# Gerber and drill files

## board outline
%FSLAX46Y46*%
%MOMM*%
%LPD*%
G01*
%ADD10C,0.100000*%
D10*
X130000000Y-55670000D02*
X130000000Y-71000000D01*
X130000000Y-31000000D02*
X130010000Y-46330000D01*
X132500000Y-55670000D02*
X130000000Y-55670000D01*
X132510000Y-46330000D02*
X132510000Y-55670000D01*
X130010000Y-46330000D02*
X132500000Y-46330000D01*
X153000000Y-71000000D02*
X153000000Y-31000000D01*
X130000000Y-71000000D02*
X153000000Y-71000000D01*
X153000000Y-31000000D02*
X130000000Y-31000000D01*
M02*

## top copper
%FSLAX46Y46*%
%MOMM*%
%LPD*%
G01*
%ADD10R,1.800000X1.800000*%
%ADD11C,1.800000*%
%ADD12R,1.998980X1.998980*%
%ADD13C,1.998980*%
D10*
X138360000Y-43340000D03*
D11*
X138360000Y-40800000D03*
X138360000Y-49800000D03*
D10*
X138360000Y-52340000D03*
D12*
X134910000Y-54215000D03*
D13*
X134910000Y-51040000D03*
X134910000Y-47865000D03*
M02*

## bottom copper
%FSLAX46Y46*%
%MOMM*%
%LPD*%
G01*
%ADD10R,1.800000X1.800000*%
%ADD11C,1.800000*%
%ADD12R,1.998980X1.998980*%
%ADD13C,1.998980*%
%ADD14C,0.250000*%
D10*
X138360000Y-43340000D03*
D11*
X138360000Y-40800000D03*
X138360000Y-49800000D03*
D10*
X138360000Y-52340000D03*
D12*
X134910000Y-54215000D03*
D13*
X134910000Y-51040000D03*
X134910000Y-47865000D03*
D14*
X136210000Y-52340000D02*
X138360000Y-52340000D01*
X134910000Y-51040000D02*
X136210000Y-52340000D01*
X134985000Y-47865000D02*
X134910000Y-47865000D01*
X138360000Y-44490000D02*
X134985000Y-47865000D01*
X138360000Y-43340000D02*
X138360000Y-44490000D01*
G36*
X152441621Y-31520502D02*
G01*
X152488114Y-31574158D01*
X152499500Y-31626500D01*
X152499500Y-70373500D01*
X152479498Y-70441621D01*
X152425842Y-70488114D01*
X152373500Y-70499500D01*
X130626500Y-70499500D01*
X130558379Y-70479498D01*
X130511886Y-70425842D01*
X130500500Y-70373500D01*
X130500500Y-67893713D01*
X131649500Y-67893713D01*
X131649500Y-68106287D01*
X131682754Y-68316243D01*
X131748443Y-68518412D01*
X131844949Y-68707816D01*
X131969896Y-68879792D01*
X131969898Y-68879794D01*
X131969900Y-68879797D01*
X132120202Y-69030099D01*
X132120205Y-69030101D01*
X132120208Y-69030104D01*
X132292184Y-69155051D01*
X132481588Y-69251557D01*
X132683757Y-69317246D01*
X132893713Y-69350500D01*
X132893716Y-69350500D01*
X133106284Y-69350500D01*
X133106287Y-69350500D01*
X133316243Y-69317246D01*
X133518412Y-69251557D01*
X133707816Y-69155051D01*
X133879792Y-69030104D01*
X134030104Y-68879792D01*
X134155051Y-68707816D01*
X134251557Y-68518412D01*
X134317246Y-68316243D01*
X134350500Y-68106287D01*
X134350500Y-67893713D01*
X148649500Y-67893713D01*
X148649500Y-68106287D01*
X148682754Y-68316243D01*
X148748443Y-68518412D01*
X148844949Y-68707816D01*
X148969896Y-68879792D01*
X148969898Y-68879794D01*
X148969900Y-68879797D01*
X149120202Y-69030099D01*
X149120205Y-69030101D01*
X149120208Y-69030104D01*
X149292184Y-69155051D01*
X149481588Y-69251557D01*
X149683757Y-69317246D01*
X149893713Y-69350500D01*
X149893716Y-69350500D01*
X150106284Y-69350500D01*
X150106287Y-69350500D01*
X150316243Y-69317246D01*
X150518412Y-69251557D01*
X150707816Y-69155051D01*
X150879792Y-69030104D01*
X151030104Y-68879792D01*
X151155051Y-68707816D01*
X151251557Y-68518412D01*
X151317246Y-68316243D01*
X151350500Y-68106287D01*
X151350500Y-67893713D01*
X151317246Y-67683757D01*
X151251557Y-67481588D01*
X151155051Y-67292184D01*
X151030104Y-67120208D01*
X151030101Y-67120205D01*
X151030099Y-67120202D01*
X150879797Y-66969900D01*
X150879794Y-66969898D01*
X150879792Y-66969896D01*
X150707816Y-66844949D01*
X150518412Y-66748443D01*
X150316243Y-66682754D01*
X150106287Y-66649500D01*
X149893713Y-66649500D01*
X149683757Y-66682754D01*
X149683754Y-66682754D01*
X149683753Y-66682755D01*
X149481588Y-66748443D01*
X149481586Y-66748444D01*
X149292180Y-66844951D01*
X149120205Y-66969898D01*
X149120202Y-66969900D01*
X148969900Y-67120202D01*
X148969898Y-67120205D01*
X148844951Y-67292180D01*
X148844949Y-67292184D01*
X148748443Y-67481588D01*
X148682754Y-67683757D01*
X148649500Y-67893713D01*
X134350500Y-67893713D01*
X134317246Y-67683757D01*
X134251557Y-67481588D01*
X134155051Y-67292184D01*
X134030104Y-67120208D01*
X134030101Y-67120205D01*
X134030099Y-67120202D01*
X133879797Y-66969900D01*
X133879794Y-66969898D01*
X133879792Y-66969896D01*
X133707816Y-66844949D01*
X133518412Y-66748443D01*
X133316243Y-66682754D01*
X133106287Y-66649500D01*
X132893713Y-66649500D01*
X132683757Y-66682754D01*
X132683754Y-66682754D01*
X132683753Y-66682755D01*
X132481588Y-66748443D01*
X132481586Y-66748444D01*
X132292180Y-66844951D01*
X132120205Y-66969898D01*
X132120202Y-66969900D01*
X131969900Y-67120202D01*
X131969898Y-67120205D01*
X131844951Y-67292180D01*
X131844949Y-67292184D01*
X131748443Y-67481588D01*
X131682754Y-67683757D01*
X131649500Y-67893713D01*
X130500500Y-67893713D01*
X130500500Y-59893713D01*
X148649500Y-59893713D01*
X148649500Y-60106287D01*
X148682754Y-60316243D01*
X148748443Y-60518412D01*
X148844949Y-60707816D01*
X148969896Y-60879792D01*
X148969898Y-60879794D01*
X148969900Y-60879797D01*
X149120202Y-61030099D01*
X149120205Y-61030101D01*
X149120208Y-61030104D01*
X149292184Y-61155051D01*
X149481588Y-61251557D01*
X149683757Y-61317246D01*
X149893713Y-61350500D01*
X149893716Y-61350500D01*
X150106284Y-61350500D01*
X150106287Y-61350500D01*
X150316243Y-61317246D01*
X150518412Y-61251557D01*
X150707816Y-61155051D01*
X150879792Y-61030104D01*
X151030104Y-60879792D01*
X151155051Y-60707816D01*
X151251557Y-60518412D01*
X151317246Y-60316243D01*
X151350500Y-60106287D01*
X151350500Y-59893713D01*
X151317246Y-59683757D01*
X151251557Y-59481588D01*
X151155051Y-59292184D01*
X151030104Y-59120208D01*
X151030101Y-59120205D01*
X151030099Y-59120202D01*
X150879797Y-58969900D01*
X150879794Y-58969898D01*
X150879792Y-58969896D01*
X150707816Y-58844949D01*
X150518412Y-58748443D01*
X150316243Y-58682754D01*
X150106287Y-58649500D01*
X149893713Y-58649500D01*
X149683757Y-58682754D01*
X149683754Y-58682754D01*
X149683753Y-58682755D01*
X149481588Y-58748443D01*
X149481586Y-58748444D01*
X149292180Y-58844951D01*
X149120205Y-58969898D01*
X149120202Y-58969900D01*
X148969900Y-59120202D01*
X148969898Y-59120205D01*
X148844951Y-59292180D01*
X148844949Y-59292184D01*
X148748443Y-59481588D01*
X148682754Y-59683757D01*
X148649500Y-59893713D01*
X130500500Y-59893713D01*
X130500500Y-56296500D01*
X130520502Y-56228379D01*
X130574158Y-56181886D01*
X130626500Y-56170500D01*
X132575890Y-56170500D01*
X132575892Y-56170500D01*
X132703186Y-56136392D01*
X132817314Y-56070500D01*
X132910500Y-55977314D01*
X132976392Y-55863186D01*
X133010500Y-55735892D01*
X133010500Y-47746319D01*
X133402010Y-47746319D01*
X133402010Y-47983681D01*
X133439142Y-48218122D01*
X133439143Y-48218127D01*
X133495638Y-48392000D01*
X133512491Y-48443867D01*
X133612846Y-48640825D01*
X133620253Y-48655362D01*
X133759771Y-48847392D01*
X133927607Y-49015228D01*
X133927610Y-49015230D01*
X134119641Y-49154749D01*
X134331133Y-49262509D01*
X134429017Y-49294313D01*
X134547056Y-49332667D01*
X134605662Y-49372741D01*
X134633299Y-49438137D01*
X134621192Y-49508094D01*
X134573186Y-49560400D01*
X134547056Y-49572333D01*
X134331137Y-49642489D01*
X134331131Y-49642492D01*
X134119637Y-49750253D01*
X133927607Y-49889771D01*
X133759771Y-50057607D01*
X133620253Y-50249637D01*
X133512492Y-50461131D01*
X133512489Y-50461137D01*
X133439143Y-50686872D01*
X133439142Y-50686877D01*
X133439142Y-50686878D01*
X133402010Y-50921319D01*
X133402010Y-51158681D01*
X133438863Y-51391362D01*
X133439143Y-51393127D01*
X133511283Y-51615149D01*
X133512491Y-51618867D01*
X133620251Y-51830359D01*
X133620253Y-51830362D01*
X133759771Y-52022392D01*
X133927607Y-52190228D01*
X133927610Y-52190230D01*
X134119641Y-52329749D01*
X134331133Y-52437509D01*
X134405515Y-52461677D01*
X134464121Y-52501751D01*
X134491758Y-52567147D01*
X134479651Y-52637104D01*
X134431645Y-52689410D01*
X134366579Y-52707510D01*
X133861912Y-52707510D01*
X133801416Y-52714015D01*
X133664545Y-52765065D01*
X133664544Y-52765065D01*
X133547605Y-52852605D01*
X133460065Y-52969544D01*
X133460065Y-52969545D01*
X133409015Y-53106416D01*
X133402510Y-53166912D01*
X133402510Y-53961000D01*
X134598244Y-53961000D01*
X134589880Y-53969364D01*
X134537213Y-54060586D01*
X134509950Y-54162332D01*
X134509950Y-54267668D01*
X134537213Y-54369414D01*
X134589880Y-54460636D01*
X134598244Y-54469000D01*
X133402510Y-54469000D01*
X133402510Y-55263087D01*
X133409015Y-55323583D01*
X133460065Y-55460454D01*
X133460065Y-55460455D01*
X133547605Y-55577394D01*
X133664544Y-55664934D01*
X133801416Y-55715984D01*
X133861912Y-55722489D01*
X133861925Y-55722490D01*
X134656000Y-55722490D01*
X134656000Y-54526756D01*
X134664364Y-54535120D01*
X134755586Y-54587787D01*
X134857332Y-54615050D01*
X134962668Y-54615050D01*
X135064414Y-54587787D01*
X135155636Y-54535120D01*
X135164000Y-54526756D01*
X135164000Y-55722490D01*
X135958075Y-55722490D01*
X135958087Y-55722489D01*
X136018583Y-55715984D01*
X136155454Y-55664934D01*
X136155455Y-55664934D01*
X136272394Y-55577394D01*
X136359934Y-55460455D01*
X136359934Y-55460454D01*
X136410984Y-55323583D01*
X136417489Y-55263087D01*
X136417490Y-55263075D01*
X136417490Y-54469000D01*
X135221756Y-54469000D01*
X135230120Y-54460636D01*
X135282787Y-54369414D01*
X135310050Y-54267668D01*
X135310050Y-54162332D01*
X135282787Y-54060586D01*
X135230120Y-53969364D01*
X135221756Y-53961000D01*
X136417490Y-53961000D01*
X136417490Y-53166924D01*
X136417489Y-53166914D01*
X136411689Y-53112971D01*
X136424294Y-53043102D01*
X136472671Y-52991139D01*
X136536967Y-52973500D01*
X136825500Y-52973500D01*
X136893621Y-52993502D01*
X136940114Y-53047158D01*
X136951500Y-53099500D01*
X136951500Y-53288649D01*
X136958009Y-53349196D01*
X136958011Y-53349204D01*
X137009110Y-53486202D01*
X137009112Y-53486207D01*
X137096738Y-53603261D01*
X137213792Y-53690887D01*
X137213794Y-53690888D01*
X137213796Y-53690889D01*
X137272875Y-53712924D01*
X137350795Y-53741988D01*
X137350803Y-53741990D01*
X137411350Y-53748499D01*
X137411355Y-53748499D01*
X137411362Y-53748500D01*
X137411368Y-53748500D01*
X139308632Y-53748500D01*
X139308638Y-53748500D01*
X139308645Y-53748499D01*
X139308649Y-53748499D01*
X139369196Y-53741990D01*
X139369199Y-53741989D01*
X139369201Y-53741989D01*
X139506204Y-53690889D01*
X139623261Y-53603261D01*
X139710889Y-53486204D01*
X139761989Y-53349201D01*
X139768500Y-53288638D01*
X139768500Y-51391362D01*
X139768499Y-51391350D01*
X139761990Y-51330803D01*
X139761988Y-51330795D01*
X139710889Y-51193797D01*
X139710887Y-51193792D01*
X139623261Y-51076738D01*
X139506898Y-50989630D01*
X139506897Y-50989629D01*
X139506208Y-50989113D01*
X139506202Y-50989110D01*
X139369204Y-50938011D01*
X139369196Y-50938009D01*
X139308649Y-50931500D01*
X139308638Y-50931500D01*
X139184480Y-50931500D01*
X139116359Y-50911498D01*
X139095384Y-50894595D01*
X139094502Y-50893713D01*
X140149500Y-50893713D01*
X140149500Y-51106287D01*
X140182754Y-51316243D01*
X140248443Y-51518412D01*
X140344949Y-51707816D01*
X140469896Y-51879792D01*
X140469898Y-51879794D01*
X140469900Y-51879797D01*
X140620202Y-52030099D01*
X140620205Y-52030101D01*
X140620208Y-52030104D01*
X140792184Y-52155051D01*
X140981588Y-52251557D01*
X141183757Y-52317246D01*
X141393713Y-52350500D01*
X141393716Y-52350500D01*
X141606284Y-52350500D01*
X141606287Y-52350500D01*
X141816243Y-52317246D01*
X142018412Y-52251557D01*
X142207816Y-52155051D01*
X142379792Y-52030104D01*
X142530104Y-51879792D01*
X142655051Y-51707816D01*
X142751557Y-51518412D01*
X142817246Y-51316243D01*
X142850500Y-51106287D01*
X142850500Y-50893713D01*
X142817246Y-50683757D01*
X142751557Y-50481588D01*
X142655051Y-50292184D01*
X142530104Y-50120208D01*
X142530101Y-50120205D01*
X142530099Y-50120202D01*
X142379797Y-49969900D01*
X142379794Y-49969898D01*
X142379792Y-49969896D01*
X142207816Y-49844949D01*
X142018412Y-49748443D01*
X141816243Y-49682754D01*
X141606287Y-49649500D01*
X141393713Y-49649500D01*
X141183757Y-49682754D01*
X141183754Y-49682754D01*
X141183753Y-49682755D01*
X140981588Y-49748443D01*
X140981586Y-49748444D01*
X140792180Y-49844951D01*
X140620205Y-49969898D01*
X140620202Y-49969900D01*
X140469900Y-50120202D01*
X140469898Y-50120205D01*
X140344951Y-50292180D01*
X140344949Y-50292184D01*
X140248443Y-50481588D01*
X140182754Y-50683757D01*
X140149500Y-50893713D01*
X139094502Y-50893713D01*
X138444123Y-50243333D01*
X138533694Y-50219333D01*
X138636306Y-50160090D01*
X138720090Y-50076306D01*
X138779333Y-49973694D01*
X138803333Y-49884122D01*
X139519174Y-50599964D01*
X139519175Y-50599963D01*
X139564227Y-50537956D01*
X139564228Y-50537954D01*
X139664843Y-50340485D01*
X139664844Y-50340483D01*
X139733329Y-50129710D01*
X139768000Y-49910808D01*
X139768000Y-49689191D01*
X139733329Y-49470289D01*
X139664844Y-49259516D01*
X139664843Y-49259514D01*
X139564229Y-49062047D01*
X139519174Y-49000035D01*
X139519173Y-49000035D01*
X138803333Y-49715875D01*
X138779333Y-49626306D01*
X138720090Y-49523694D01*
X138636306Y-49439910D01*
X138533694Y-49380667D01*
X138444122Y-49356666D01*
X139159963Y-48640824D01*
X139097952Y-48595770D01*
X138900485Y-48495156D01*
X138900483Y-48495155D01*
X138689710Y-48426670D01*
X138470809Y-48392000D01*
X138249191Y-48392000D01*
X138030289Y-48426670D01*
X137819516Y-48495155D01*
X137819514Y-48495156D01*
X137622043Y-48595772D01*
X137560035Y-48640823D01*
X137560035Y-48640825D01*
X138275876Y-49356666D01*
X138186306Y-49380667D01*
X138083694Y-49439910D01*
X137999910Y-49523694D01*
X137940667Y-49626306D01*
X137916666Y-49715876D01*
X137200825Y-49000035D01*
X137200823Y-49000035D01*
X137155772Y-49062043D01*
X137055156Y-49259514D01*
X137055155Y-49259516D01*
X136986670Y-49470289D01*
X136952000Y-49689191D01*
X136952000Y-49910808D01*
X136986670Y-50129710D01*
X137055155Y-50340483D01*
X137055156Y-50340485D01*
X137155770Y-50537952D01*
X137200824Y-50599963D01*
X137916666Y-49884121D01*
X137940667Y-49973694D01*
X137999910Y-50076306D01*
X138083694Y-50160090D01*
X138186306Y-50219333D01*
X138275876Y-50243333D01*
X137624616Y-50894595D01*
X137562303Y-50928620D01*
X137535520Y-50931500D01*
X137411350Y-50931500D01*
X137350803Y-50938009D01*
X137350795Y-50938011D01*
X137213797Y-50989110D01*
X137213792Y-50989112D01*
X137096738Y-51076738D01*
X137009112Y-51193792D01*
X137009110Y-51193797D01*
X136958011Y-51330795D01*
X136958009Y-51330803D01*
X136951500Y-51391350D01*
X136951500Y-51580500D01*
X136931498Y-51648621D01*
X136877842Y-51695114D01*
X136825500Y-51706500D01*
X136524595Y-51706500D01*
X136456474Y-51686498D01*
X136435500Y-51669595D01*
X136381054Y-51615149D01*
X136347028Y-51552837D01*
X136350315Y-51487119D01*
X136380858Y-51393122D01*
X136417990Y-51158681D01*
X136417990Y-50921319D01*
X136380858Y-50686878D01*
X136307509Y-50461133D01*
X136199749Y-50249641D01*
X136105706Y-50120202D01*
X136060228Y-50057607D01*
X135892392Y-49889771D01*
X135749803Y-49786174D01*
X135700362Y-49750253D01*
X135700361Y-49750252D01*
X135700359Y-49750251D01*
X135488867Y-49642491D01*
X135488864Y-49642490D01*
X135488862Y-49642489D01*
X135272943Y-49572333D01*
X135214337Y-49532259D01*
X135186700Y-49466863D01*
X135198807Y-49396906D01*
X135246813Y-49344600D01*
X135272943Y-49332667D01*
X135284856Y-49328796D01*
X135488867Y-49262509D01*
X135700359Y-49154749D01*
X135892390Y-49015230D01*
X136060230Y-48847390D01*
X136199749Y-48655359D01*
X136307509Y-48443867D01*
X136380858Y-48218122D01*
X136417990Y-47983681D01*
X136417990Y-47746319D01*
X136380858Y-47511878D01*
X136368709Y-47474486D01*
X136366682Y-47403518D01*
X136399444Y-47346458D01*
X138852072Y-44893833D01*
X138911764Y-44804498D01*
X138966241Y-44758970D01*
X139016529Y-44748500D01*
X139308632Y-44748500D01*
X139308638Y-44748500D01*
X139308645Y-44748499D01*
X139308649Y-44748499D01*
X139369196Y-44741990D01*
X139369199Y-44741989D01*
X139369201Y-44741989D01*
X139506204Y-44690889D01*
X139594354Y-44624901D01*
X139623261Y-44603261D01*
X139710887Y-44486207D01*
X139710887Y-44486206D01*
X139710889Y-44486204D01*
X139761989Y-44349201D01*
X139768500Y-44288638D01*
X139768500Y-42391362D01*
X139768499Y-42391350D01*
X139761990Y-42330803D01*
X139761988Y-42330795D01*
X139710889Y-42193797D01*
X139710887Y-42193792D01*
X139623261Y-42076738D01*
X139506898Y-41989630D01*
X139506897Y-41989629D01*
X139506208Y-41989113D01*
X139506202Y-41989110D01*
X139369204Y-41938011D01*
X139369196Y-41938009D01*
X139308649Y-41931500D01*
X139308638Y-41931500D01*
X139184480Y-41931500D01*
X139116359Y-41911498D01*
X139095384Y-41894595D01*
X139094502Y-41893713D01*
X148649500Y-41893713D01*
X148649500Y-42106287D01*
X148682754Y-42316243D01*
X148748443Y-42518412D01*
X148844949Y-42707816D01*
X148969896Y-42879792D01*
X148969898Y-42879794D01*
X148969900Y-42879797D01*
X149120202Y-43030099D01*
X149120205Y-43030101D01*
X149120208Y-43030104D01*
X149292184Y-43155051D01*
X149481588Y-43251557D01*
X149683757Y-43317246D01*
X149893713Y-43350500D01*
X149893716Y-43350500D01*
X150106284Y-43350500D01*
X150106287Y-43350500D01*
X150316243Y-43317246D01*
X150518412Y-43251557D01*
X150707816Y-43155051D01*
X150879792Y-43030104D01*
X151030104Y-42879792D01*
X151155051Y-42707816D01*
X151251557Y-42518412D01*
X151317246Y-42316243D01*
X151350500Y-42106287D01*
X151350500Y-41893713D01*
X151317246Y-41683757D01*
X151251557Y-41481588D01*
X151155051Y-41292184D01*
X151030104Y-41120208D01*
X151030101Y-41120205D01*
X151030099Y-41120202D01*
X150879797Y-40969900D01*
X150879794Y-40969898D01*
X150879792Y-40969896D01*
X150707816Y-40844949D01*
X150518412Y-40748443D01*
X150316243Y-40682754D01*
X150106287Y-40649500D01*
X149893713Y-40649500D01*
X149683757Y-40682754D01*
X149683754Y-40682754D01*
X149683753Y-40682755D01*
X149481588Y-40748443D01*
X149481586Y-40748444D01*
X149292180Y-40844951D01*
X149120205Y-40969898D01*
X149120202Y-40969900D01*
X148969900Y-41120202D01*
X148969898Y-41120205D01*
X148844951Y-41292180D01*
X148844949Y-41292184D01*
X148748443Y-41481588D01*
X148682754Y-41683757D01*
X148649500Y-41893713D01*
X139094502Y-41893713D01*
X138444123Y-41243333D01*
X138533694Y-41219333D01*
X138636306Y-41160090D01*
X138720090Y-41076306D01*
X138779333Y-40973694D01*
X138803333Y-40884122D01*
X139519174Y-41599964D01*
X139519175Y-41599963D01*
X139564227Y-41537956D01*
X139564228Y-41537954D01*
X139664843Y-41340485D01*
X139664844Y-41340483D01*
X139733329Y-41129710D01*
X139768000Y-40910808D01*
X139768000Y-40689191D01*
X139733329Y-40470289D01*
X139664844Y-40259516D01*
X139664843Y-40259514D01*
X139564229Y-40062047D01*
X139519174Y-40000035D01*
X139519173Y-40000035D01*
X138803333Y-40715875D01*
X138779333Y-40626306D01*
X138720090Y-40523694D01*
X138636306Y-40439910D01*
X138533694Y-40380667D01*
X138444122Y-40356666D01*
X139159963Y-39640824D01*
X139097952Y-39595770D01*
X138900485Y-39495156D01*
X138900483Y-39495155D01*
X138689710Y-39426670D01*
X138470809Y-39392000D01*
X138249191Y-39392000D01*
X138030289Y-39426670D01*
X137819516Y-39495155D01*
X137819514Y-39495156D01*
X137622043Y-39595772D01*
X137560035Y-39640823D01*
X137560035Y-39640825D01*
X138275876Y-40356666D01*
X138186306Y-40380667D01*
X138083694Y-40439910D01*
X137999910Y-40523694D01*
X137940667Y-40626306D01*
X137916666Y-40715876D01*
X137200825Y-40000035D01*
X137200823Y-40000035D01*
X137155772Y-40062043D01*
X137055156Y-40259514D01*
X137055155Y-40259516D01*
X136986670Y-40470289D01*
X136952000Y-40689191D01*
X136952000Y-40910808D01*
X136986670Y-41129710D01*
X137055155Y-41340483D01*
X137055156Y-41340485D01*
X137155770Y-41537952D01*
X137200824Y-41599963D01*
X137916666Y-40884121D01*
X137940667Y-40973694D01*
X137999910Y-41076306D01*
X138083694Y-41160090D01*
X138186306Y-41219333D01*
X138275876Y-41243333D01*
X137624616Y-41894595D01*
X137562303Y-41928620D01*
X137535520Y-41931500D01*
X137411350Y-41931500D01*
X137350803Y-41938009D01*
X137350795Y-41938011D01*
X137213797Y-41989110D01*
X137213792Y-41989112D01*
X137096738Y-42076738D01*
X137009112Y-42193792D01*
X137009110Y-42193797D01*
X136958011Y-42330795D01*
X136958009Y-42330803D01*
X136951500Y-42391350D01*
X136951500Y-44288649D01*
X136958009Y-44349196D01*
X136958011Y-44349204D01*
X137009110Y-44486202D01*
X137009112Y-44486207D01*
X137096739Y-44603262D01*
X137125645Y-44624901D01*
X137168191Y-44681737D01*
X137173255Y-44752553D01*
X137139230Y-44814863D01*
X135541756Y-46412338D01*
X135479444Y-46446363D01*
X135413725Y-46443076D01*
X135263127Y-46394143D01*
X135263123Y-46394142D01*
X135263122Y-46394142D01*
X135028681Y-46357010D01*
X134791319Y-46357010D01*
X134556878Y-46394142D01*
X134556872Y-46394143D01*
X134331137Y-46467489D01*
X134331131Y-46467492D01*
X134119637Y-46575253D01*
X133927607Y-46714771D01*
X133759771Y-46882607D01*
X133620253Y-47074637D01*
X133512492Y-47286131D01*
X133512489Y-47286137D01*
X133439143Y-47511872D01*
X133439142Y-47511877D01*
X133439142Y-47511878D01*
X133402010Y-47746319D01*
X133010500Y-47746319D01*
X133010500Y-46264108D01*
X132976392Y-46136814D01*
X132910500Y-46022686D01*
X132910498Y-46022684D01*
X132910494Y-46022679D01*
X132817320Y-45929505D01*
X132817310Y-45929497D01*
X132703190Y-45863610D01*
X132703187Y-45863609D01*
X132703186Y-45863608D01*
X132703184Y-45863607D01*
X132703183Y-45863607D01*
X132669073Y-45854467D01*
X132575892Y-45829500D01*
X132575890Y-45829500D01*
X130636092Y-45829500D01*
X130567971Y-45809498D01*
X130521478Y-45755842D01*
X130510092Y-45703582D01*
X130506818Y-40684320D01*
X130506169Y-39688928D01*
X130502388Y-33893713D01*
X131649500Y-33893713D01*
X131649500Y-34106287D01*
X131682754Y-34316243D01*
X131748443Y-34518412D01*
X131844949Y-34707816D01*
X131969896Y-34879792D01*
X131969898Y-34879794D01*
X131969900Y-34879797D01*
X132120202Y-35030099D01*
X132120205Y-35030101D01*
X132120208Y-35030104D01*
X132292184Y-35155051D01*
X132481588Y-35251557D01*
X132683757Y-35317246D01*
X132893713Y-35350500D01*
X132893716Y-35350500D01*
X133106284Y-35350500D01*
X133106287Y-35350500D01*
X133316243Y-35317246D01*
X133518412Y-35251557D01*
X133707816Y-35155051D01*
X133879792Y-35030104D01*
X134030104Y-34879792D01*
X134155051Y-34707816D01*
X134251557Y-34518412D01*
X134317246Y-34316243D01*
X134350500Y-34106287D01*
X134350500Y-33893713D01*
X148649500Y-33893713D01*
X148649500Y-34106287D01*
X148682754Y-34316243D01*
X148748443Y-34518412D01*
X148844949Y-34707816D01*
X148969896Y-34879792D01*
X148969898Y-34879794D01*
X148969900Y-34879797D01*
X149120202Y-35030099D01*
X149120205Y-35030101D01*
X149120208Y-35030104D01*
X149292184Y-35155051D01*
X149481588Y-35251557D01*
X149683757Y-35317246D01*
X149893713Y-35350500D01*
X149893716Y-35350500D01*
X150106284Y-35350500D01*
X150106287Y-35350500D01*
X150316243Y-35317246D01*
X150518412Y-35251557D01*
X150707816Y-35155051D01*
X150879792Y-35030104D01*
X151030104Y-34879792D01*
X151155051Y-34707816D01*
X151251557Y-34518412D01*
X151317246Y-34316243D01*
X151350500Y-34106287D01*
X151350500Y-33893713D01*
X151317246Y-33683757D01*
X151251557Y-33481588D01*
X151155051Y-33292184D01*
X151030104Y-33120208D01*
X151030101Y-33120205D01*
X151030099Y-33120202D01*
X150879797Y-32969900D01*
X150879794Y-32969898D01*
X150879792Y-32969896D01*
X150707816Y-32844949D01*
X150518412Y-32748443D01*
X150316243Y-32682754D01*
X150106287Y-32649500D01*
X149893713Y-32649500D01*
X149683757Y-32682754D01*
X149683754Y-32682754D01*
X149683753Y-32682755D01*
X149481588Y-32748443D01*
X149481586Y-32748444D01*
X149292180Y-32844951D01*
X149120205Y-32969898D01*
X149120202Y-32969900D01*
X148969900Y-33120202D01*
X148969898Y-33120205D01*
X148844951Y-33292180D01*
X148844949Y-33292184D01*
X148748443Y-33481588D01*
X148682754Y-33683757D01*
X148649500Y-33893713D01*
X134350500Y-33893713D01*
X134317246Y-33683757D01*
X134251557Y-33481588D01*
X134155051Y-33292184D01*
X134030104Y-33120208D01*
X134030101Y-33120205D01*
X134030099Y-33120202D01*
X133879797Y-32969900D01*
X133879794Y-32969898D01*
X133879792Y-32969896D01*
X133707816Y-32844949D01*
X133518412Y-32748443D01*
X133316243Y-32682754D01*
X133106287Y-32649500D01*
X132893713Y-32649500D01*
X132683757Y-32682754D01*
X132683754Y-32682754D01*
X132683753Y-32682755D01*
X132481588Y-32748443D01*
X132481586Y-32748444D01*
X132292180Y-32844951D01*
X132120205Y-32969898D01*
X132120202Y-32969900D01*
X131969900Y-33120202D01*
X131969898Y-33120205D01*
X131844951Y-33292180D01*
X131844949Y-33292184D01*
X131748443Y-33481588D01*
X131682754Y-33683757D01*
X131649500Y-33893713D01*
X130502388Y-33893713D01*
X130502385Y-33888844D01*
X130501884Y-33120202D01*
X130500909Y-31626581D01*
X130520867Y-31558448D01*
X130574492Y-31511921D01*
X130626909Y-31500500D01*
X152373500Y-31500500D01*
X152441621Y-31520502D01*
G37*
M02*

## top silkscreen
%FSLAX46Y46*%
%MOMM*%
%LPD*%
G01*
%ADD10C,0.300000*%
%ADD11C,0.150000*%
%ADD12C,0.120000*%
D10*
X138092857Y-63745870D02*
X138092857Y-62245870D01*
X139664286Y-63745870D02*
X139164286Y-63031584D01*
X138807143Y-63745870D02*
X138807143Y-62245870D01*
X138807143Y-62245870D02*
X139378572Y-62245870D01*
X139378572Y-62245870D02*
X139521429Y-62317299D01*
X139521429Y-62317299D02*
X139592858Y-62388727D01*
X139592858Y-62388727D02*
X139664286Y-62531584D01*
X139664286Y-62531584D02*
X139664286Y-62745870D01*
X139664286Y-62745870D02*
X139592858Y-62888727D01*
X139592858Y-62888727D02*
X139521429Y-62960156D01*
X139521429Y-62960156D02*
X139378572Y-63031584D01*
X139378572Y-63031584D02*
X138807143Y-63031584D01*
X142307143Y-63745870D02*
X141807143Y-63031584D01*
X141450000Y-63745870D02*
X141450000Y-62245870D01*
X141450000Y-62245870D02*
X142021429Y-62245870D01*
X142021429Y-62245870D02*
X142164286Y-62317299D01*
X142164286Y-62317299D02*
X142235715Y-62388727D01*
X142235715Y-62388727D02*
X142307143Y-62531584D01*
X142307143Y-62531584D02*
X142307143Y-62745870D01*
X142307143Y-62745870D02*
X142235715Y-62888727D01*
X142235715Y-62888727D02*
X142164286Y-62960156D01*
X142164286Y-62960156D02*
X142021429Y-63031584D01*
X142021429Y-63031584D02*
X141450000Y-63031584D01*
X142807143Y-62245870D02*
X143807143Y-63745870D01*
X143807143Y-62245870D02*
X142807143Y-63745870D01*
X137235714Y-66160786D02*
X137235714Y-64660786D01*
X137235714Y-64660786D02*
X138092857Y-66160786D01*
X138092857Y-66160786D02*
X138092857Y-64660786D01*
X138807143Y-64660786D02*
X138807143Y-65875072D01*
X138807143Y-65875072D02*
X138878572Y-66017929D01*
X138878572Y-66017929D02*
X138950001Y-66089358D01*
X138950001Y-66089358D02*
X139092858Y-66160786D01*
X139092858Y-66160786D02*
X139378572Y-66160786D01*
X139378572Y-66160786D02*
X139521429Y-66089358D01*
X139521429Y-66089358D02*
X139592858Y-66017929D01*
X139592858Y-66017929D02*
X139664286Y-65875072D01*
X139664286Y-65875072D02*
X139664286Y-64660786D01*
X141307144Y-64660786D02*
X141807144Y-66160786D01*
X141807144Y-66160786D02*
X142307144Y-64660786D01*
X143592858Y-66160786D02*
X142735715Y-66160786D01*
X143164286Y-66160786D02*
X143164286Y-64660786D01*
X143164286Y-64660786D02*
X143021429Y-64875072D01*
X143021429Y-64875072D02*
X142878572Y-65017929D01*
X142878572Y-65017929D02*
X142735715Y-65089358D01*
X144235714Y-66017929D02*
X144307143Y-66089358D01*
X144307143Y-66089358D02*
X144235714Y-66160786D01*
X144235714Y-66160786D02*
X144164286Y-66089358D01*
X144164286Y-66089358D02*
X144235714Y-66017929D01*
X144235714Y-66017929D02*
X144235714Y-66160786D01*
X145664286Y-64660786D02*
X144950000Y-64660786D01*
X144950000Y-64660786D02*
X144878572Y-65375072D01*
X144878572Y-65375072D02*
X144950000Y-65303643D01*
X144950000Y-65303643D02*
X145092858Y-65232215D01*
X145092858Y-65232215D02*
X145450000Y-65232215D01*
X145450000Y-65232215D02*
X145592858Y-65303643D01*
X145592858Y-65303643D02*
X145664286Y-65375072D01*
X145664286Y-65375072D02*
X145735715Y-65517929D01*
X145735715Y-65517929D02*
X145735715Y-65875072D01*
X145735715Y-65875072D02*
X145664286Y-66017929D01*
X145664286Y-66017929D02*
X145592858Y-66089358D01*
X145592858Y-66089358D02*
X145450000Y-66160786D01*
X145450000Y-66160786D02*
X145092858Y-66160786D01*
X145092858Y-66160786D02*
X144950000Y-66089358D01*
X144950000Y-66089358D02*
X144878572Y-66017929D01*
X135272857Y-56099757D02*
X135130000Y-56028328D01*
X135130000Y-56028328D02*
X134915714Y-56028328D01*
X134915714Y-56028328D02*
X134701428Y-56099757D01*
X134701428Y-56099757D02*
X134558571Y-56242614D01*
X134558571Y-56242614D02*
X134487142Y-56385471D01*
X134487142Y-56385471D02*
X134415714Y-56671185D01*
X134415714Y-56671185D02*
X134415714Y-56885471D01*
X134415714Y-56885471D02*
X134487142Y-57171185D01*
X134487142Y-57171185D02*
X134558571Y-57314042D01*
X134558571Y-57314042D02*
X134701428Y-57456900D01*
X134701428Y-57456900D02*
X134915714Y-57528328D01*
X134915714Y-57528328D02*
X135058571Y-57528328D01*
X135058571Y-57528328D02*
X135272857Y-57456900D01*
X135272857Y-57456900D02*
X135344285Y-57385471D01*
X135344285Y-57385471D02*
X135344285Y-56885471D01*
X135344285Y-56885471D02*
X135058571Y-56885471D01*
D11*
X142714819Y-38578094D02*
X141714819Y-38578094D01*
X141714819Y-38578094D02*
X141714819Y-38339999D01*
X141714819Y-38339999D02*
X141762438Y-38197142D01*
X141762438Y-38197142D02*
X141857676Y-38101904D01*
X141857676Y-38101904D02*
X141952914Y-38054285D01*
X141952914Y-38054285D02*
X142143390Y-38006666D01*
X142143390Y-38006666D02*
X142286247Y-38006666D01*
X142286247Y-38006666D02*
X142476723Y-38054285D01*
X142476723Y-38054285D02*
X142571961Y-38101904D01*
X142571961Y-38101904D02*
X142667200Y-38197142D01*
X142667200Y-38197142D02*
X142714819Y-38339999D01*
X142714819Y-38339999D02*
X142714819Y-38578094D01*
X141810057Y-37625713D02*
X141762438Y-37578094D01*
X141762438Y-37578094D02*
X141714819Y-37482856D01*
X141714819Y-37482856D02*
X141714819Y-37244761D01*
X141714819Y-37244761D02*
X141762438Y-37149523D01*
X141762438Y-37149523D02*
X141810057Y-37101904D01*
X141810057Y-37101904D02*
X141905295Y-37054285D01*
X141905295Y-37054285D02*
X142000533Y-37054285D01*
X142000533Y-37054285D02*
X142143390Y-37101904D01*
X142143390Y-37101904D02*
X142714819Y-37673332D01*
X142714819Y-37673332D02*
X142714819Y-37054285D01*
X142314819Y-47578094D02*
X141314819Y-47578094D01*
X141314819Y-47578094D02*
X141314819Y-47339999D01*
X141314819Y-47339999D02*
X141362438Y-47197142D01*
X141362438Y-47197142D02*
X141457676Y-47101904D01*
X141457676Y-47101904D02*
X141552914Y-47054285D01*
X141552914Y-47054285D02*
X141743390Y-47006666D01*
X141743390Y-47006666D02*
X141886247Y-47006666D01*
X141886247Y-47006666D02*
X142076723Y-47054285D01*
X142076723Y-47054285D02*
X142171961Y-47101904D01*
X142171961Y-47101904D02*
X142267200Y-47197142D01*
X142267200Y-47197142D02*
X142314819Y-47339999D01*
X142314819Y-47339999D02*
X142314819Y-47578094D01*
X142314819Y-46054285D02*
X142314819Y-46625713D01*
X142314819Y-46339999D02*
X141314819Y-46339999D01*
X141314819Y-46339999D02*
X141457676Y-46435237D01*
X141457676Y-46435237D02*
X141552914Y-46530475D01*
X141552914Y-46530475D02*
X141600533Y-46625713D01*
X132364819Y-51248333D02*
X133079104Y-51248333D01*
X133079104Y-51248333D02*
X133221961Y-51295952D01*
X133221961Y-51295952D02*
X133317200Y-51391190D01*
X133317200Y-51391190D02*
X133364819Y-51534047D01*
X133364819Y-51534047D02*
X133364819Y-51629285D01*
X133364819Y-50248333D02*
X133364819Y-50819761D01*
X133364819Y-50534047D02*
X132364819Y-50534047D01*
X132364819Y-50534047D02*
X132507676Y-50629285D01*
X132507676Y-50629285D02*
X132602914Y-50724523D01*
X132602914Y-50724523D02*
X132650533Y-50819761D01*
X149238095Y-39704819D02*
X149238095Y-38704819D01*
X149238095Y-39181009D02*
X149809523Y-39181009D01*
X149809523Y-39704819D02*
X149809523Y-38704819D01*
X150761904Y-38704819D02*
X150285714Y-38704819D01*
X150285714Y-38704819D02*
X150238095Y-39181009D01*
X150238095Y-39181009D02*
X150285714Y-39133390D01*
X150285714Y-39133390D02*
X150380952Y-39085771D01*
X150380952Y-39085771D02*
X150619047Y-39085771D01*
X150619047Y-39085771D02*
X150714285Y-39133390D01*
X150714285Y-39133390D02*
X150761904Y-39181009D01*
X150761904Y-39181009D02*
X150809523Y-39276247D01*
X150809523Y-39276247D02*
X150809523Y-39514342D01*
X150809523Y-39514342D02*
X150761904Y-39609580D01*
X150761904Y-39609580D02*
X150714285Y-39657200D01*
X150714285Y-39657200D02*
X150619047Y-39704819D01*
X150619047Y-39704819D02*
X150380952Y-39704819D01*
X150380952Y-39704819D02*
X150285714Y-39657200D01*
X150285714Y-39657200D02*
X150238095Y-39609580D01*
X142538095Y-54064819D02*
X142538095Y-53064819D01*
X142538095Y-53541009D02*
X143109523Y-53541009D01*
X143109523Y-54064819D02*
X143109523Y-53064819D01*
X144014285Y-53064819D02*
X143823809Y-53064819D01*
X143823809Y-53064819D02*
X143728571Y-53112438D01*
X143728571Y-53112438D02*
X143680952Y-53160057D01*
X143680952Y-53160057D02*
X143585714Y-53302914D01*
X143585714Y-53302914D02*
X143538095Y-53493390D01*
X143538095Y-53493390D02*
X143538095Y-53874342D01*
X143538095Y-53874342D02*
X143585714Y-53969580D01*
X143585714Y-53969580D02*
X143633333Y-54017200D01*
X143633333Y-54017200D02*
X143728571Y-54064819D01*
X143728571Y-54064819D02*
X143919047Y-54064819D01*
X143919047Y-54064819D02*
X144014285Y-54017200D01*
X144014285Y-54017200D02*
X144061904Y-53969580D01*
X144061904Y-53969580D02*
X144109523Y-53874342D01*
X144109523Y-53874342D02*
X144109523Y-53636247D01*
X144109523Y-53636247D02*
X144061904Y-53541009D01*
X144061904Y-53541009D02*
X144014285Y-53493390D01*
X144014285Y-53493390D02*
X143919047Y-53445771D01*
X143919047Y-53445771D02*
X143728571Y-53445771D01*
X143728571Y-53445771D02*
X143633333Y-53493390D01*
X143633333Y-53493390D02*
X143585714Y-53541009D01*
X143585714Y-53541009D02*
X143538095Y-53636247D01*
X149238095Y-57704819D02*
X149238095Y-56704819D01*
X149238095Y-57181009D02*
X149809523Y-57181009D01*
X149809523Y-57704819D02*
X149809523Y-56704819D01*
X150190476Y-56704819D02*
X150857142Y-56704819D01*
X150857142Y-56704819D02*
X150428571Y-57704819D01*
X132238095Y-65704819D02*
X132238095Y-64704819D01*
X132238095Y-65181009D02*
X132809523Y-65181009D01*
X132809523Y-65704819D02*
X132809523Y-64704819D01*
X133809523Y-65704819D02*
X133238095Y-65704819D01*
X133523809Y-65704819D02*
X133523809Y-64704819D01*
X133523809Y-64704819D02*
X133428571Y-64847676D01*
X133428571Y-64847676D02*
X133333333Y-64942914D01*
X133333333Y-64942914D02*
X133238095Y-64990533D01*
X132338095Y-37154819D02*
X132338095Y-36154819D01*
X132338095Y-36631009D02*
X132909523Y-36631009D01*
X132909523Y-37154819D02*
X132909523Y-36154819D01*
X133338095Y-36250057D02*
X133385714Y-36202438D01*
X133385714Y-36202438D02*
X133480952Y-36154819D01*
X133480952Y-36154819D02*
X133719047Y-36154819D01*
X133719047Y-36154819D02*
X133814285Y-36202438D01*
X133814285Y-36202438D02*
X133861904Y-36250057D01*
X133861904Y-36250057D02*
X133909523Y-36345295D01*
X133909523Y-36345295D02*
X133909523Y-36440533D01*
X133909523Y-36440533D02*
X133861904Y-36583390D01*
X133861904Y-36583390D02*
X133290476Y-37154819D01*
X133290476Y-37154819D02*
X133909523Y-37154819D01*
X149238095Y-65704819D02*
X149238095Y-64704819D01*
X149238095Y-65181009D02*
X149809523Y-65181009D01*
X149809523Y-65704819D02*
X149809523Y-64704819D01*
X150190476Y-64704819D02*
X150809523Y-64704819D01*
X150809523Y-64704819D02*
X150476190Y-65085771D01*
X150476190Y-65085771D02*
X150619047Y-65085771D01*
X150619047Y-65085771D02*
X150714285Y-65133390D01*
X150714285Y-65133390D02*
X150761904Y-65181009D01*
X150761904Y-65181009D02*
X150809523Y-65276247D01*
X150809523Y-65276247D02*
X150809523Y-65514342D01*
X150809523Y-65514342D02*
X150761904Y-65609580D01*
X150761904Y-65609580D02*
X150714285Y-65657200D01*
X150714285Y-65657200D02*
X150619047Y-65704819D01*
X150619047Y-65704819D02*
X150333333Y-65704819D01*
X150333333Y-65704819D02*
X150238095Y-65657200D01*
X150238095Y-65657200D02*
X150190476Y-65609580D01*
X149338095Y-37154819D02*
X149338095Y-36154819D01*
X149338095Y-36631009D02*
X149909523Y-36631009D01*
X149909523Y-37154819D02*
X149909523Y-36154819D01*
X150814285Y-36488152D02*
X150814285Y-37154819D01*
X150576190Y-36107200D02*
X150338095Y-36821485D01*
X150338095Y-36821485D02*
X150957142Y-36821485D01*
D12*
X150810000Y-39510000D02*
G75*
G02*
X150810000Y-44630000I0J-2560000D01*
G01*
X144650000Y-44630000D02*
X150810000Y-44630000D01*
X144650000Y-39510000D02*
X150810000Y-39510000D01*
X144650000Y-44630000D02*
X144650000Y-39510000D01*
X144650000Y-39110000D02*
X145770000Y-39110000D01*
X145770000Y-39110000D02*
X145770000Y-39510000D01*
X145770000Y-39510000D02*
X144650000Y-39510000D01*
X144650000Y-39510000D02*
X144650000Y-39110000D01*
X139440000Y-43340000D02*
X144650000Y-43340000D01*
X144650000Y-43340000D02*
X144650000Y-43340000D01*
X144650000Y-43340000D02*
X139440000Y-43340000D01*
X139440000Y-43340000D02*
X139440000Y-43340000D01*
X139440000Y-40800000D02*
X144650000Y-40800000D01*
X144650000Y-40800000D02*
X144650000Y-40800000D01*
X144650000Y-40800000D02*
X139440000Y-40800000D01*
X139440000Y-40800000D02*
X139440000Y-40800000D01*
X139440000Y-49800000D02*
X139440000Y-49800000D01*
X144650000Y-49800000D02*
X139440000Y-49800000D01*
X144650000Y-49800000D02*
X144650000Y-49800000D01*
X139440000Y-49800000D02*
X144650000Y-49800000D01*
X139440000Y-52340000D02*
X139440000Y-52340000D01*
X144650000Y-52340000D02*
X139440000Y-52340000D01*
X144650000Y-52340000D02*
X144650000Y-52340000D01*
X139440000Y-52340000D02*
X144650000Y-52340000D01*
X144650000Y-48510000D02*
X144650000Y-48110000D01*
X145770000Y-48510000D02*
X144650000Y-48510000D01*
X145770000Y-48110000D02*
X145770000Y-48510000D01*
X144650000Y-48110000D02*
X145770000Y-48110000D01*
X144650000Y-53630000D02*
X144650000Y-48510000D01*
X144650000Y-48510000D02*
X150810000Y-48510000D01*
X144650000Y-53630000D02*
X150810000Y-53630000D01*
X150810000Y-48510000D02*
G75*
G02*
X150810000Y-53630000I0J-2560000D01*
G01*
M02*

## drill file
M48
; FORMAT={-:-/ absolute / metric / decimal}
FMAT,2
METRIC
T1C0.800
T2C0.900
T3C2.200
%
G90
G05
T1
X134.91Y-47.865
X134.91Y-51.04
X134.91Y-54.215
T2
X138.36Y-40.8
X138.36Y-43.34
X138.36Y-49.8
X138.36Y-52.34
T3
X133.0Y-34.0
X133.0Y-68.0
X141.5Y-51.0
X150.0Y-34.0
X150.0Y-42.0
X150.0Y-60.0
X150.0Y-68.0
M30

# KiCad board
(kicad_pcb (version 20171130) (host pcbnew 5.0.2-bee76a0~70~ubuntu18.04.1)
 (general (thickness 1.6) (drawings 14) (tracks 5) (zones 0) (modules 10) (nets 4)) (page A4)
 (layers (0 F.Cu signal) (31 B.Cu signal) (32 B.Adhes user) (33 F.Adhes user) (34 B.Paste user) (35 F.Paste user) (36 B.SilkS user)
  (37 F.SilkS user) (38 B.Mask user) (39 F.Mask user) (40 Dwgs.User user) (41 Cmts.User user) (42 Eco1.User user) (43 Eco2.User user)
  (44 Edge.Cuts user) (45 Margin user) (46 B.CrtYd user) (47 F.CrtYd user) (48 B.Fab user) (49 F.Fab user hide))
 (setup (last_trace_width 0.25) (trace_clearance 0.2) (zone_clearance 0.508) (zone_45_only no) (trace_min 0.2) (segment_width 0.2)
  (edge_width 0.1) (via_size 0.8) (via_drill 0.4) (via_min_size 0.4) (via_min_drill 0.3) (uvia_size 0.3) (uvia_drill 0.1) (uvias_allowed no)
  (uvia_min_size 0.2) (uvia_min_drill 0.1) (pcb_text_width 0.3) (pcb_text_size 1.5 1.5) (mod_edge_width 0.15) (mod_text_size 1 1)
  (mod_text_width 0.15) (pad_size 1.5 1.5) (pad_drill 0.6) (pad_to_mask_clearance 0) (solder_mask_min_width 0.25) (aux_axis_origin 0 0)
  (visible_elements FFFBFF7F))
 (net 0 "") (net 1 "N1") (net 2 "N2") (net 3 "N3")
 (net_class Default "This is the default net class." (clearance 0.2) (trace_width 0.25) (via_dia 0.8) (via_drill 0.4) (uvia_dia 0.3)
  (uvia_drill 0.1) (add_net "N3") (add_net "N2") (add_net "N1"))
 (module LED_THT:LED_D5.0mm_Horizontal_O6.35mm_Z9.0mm (layer F.Cu) (at 138.36 43.34 90)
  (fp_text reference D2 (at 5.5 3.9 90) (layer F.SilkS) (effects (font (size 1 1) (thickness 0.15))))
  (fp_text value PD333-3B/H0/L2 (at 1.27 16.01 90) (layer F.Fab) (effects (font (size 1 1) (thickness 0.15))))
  (fp_arc (start 1.27 12.45) (end -1.29 12.45) (angle -180) (layer F.SilkS) (width 0.12))
  (fp_line (start -1.29 6.29) (end -1.29 12.45) (layer F.SilkS) (width 0.12))
  (fp_line (start 3.83 6.29) (end 3.83 12.45) (layer F.SilkS) (width 0.12))
  (fp_line (start -1.29 6.29) (end 3.83 6.29) (layer F.SilkS) (width 0.12))
  (fp_line (start 4.23 6.29) (end 4.23 7.41) (layer F.SilkS) (width 0.12))
  (fp_line (start 4.23 7.41) (end 3.83 7.41) (layer F.SilkS) (width 0.12))
  (fp_line (start 3.83 7.41) (end 3.83 6.29) (layer F.SilkS) (width 0.12))
  (fp_line (start 3.83 6.29) (end 4.23 6.29) (layer F.SilkS) (width 0.12))
  (fp_line (start 0 1.08) (end 0 6.29) (layer F.SilkS) (width 0.12))
  (fp_line (start 0 6.29) (end 0 6.29) (layer F.SilkS) (width 0.12))
  (fp_line (start 0 6.29) (end 0 1.08) (layer F.SilkS) (width 0.12))
  (fp_line (start 0 1.08) (end 0 1.08) (layer F.SilkS) (width 0.12))
  (fp_line (start 2.54 1.08) (end 2.54 6.29) (layer F.SilkS) (width 0.12))
  (fp_line (start 2.54 6.29) (end 2.54 6.29) (layer F.SilkS) (width 0.12))
  (fp_line (start 2.54 6.29) (end 2.54 1.08) (layer F.SilkS) (width 0.12))
  (fp_line (start 2.54 1.08) (end 2.54 1.08) (layer F.SilkS) (width 0.12))
  (pad 1 thru_hole rect (at 0 0 90) (size 1.8 1.8) (drill 0.9) (layers *.Cu *.Mask) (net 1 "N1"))
  (pad 2 thru_hole circle (at 2.54 0 90) (size 1.8 1.8) (drill 0.9) (layers *.Cu *.Mask) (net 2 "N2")))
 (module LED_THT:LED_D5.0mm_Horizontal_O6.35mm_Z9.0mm (layer F.Cu) (at 138.36 52.34 90)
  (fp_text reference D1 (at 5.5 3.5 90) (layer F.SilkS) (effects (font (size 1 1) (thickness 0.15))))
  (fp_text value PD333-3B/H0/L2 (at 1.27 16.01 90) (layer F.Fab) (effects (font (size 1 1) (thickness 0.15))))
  (fp_line (start 2.54 1.08) (end 2.54 1.08) (layer F.SilkS) (width 0.12))
  (fp_line (start 2.54 6.29) (end 2.54 1.08) (layer F.SilkS) (width 0.12))
  (fp_line (start 2.54 6.29) (end 2.54 6.29) (layer F.SilkS) (width 0.12))
  (fp_line (start 2.54 1.08) (end 2.54 6.29) (layer F.SilkS) (width 0.12))
  (fp_line (start 0 1.08) (end 0 1.08) (layer F.SilkS) (width 0.12))
  (fp_line (start 0 6.29) (end 0 1.08) (layer F.SilkS) (width 0.12))
  (fp_line (start 0 6.29) (end 0 6.29) (layer F.SilkS) (width 0.12))
  (fp_line (start 0 1.08) (end 0 6.29) (layer F.SilkS) (width 0.12))
  (fp_line (start 3.83 6.29) (end 4.23 6.29) (layer F.SilkS) (width 0.12))
  (fp_line (start 3.83 7.41) (end 3.83 6.29) (layer F.SilkS) (width 0.12))
  (fp_line (start 4.23 7.41) (end 3.83 7.41) (layer F.SilkS) (width 0.12))
  (fp_line (start 4.23 6.29) (end 4.23 7.41) (layer F.SilkS) (width 0.12))
  (fp_line (start -1.29 6.29) (end 3.83 6.29) (layer F.SilkS) (width 0.12))
  (fp_line (start 3.83 6.29) (end 3.83 12.45) (layer F.SilkS) (width 0.12))
  (fp_line (start -1.29 6.29) (end -1.29 12.45) (layer F.SilkS) (width 0.12))
  (fp_arc (start 1.27 12.45) (end -1.29 12.45) (angle -180) (layer F.SilkS) (width 0.12))
  (pad 2 thru_hole circle (at 2.54 0 90) (size 1.8 1.8) (drill 0.9) (layers *.Cu *.Mask) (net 2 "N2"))
  (pad 1 thru_hole rect (at 0 0 90) (size 1.8 1.8) (drill 0.9) (layers *.Cu *.Mask) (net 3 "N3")))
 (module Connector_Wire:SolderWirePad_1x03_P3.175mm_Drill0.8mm (layer F.Cu) (at 134.91 54.215 90)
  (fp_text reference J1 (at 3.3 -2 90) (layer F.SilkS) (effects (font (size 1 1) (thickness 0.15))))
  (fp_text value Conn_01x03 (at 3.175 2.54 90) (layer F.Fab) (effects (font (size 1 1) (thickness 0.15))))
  (pad 1 thru_hole rect (at 0 0 90) (size 1.99898 1.99898) (drill 0.8001) (layers *.Cu *.Mask) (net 2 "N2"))
  (pad 2 thru_hole circle (at 3.175 0 90) (size 1.99898 1.99898) (drill 0.8001) (layers *.Cu *.Mask) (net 3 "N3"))
  (pad 3 thru_hole circle (at 6.35 0 90) (size 1.99898 1.99898) (drill 0.8001) (layers *.Cu *.Mask) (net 1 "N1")))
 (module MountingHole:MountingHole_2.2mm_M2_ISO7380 (layer F.Cu) (at 150 42)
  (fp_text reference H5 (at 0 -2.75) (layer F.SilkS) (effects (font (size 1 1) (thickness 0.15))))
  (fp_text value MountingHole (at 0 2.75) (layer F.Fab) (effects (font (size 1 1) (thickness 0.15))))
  (pad 1 np_thru_hole circle (at 0 0) (size 2.2 2.2) (drill 2.2) (layers *.Cu *.Mask)))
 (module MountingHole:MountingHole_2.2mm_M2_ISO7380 (layer F.Cu) (at 141.5 51)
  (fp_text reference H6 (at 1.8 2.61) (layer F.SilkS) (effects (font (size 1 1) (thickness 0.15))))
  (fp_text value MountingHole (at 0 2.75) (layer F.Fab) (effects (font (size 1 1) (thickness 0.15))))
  (pad 1 np_thru_hole circle (at 0 0) (size 2.2 2.2) (drill 2.2) (layers *.Cu *.Mask)))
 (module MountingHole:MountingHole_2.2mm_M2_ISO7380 (layer F.Cu) (at 150 60)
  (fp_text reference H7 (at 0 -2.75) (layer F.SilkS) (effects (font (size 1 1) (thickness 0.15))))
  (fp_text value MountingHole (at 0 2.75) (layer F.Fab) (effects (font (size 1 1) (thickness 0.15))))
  (pad 1 np_thru_hole circle (at 0 0) (size 2.2 2.2) (drill 2.2) (layers *.Cu *.Mask)))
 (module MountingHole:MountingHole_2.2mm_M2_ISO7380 (layer F.Cu) (at 133 68)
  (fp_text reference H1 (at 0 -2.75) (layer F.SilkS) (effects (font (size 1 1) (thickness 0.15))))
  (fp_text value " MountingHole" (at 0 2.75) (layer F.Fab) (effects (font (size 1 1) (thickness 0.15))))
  (pad 1 np_thru_hole circle (at 0 0) (size 2.2 2.2) (drill 2.2) (layers *.Cu *.Mask)))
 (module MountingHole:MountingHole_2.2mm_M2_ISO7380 (layer F.Cu) (at 133 34)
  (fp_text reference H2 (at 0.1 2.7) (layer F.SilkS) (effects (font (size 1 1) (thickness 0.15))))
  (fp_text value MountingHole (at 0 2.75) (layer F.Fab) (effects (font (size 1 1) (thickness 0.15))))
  (pad 1 np_thru_hole circle (at 0 0) (size 2.2 2.2) (drill 2.2) (layers *.Cu *.Mask)))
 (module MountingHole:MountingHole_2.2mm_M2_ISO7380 (layer F.Cu) (at 150 68)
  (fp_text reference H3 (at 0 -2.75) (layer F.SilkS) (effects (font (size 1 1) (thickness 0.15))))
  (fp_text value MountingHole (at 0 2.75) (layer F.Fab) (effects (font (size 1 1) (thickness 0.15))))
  (pad 1 np_thru_hole circle (at 0 0) (size 2.2 2.2) (drill 2.2) (layers *.Cu *.Mask)))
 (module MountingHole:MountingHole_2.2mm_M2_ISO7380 (layer F.Cu) (at 150 34)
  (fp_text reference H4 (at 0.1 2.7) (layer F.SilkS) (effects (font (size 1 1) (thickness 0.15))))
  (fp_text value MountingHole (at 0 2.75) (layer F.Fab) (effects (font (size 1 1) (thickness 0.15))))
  (pad 1 np_thru_hole circle (at 0 0) (size 2.2 2.2) (drill 2.2) (layers *.Cu *.Mask)))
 (gr_line (start 130 55.67) (end 130 71) (layer Edge.Cuts) (width 0.1))
 (gr_line (start 130 31) (end 130.01 46.33) (layer Edge.Cuts) (width 0.1))
 (gr_line (start 132.5 55.67) (end 130 55.67) (layer Edge.Cuts) (width 0.1))
 (gr_line (start 132.51 46.33) (end 132.51 55.67) (layer Edge.Cuts) (width 0.1))
 (gr_line (start 130.01 46.33) (end 132.5 46.33) (layer Edge.Cuts) (width 0.1))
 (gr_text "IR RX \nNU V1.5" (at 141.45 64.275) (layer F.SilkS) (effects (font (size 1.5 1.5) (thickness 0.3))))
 (gr_line (start 153 71) (end 153 31) (layer Edge.Cuts) (width 0.1))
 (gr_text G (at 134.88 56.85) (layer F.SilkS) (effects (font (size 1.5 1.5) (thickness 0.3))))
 (gr_line (start 130 71) (end 153 71) (layer Edge.Cuts) (width 0.1))
 (gr_line (start 153 31) (end 130 31) (layer Edge.Cuts) (width 0.1))
 (segment (start 136.21 52.34) (end 138.36 52.34) (width 0.25) (layer B.Cu) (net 3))
 (segment (start 134.91 51.04) (end 136.21 52.34) (width 0.25) (layer B.Cu) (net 3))
 (segment (start 134.985 47.865) (end 134.91 47.865) (width 0.25) (layer B.Cu) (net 1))
 (segment (start 138.36 44.49) (end 134.985 47.865) (width 0.25) (layer B.Cu) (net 1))
 (segment (start 138.36 43.34) (end 138.36 44.49) (width 0.25) (layer B.Cu) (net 1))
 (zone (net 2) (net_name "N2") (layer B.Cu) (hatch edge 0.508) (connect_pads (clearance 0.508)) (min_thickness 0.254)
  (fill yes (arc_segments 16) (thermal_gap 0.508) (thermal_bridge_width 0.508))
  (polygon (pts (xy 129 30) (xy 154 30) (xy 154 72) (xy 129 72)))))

